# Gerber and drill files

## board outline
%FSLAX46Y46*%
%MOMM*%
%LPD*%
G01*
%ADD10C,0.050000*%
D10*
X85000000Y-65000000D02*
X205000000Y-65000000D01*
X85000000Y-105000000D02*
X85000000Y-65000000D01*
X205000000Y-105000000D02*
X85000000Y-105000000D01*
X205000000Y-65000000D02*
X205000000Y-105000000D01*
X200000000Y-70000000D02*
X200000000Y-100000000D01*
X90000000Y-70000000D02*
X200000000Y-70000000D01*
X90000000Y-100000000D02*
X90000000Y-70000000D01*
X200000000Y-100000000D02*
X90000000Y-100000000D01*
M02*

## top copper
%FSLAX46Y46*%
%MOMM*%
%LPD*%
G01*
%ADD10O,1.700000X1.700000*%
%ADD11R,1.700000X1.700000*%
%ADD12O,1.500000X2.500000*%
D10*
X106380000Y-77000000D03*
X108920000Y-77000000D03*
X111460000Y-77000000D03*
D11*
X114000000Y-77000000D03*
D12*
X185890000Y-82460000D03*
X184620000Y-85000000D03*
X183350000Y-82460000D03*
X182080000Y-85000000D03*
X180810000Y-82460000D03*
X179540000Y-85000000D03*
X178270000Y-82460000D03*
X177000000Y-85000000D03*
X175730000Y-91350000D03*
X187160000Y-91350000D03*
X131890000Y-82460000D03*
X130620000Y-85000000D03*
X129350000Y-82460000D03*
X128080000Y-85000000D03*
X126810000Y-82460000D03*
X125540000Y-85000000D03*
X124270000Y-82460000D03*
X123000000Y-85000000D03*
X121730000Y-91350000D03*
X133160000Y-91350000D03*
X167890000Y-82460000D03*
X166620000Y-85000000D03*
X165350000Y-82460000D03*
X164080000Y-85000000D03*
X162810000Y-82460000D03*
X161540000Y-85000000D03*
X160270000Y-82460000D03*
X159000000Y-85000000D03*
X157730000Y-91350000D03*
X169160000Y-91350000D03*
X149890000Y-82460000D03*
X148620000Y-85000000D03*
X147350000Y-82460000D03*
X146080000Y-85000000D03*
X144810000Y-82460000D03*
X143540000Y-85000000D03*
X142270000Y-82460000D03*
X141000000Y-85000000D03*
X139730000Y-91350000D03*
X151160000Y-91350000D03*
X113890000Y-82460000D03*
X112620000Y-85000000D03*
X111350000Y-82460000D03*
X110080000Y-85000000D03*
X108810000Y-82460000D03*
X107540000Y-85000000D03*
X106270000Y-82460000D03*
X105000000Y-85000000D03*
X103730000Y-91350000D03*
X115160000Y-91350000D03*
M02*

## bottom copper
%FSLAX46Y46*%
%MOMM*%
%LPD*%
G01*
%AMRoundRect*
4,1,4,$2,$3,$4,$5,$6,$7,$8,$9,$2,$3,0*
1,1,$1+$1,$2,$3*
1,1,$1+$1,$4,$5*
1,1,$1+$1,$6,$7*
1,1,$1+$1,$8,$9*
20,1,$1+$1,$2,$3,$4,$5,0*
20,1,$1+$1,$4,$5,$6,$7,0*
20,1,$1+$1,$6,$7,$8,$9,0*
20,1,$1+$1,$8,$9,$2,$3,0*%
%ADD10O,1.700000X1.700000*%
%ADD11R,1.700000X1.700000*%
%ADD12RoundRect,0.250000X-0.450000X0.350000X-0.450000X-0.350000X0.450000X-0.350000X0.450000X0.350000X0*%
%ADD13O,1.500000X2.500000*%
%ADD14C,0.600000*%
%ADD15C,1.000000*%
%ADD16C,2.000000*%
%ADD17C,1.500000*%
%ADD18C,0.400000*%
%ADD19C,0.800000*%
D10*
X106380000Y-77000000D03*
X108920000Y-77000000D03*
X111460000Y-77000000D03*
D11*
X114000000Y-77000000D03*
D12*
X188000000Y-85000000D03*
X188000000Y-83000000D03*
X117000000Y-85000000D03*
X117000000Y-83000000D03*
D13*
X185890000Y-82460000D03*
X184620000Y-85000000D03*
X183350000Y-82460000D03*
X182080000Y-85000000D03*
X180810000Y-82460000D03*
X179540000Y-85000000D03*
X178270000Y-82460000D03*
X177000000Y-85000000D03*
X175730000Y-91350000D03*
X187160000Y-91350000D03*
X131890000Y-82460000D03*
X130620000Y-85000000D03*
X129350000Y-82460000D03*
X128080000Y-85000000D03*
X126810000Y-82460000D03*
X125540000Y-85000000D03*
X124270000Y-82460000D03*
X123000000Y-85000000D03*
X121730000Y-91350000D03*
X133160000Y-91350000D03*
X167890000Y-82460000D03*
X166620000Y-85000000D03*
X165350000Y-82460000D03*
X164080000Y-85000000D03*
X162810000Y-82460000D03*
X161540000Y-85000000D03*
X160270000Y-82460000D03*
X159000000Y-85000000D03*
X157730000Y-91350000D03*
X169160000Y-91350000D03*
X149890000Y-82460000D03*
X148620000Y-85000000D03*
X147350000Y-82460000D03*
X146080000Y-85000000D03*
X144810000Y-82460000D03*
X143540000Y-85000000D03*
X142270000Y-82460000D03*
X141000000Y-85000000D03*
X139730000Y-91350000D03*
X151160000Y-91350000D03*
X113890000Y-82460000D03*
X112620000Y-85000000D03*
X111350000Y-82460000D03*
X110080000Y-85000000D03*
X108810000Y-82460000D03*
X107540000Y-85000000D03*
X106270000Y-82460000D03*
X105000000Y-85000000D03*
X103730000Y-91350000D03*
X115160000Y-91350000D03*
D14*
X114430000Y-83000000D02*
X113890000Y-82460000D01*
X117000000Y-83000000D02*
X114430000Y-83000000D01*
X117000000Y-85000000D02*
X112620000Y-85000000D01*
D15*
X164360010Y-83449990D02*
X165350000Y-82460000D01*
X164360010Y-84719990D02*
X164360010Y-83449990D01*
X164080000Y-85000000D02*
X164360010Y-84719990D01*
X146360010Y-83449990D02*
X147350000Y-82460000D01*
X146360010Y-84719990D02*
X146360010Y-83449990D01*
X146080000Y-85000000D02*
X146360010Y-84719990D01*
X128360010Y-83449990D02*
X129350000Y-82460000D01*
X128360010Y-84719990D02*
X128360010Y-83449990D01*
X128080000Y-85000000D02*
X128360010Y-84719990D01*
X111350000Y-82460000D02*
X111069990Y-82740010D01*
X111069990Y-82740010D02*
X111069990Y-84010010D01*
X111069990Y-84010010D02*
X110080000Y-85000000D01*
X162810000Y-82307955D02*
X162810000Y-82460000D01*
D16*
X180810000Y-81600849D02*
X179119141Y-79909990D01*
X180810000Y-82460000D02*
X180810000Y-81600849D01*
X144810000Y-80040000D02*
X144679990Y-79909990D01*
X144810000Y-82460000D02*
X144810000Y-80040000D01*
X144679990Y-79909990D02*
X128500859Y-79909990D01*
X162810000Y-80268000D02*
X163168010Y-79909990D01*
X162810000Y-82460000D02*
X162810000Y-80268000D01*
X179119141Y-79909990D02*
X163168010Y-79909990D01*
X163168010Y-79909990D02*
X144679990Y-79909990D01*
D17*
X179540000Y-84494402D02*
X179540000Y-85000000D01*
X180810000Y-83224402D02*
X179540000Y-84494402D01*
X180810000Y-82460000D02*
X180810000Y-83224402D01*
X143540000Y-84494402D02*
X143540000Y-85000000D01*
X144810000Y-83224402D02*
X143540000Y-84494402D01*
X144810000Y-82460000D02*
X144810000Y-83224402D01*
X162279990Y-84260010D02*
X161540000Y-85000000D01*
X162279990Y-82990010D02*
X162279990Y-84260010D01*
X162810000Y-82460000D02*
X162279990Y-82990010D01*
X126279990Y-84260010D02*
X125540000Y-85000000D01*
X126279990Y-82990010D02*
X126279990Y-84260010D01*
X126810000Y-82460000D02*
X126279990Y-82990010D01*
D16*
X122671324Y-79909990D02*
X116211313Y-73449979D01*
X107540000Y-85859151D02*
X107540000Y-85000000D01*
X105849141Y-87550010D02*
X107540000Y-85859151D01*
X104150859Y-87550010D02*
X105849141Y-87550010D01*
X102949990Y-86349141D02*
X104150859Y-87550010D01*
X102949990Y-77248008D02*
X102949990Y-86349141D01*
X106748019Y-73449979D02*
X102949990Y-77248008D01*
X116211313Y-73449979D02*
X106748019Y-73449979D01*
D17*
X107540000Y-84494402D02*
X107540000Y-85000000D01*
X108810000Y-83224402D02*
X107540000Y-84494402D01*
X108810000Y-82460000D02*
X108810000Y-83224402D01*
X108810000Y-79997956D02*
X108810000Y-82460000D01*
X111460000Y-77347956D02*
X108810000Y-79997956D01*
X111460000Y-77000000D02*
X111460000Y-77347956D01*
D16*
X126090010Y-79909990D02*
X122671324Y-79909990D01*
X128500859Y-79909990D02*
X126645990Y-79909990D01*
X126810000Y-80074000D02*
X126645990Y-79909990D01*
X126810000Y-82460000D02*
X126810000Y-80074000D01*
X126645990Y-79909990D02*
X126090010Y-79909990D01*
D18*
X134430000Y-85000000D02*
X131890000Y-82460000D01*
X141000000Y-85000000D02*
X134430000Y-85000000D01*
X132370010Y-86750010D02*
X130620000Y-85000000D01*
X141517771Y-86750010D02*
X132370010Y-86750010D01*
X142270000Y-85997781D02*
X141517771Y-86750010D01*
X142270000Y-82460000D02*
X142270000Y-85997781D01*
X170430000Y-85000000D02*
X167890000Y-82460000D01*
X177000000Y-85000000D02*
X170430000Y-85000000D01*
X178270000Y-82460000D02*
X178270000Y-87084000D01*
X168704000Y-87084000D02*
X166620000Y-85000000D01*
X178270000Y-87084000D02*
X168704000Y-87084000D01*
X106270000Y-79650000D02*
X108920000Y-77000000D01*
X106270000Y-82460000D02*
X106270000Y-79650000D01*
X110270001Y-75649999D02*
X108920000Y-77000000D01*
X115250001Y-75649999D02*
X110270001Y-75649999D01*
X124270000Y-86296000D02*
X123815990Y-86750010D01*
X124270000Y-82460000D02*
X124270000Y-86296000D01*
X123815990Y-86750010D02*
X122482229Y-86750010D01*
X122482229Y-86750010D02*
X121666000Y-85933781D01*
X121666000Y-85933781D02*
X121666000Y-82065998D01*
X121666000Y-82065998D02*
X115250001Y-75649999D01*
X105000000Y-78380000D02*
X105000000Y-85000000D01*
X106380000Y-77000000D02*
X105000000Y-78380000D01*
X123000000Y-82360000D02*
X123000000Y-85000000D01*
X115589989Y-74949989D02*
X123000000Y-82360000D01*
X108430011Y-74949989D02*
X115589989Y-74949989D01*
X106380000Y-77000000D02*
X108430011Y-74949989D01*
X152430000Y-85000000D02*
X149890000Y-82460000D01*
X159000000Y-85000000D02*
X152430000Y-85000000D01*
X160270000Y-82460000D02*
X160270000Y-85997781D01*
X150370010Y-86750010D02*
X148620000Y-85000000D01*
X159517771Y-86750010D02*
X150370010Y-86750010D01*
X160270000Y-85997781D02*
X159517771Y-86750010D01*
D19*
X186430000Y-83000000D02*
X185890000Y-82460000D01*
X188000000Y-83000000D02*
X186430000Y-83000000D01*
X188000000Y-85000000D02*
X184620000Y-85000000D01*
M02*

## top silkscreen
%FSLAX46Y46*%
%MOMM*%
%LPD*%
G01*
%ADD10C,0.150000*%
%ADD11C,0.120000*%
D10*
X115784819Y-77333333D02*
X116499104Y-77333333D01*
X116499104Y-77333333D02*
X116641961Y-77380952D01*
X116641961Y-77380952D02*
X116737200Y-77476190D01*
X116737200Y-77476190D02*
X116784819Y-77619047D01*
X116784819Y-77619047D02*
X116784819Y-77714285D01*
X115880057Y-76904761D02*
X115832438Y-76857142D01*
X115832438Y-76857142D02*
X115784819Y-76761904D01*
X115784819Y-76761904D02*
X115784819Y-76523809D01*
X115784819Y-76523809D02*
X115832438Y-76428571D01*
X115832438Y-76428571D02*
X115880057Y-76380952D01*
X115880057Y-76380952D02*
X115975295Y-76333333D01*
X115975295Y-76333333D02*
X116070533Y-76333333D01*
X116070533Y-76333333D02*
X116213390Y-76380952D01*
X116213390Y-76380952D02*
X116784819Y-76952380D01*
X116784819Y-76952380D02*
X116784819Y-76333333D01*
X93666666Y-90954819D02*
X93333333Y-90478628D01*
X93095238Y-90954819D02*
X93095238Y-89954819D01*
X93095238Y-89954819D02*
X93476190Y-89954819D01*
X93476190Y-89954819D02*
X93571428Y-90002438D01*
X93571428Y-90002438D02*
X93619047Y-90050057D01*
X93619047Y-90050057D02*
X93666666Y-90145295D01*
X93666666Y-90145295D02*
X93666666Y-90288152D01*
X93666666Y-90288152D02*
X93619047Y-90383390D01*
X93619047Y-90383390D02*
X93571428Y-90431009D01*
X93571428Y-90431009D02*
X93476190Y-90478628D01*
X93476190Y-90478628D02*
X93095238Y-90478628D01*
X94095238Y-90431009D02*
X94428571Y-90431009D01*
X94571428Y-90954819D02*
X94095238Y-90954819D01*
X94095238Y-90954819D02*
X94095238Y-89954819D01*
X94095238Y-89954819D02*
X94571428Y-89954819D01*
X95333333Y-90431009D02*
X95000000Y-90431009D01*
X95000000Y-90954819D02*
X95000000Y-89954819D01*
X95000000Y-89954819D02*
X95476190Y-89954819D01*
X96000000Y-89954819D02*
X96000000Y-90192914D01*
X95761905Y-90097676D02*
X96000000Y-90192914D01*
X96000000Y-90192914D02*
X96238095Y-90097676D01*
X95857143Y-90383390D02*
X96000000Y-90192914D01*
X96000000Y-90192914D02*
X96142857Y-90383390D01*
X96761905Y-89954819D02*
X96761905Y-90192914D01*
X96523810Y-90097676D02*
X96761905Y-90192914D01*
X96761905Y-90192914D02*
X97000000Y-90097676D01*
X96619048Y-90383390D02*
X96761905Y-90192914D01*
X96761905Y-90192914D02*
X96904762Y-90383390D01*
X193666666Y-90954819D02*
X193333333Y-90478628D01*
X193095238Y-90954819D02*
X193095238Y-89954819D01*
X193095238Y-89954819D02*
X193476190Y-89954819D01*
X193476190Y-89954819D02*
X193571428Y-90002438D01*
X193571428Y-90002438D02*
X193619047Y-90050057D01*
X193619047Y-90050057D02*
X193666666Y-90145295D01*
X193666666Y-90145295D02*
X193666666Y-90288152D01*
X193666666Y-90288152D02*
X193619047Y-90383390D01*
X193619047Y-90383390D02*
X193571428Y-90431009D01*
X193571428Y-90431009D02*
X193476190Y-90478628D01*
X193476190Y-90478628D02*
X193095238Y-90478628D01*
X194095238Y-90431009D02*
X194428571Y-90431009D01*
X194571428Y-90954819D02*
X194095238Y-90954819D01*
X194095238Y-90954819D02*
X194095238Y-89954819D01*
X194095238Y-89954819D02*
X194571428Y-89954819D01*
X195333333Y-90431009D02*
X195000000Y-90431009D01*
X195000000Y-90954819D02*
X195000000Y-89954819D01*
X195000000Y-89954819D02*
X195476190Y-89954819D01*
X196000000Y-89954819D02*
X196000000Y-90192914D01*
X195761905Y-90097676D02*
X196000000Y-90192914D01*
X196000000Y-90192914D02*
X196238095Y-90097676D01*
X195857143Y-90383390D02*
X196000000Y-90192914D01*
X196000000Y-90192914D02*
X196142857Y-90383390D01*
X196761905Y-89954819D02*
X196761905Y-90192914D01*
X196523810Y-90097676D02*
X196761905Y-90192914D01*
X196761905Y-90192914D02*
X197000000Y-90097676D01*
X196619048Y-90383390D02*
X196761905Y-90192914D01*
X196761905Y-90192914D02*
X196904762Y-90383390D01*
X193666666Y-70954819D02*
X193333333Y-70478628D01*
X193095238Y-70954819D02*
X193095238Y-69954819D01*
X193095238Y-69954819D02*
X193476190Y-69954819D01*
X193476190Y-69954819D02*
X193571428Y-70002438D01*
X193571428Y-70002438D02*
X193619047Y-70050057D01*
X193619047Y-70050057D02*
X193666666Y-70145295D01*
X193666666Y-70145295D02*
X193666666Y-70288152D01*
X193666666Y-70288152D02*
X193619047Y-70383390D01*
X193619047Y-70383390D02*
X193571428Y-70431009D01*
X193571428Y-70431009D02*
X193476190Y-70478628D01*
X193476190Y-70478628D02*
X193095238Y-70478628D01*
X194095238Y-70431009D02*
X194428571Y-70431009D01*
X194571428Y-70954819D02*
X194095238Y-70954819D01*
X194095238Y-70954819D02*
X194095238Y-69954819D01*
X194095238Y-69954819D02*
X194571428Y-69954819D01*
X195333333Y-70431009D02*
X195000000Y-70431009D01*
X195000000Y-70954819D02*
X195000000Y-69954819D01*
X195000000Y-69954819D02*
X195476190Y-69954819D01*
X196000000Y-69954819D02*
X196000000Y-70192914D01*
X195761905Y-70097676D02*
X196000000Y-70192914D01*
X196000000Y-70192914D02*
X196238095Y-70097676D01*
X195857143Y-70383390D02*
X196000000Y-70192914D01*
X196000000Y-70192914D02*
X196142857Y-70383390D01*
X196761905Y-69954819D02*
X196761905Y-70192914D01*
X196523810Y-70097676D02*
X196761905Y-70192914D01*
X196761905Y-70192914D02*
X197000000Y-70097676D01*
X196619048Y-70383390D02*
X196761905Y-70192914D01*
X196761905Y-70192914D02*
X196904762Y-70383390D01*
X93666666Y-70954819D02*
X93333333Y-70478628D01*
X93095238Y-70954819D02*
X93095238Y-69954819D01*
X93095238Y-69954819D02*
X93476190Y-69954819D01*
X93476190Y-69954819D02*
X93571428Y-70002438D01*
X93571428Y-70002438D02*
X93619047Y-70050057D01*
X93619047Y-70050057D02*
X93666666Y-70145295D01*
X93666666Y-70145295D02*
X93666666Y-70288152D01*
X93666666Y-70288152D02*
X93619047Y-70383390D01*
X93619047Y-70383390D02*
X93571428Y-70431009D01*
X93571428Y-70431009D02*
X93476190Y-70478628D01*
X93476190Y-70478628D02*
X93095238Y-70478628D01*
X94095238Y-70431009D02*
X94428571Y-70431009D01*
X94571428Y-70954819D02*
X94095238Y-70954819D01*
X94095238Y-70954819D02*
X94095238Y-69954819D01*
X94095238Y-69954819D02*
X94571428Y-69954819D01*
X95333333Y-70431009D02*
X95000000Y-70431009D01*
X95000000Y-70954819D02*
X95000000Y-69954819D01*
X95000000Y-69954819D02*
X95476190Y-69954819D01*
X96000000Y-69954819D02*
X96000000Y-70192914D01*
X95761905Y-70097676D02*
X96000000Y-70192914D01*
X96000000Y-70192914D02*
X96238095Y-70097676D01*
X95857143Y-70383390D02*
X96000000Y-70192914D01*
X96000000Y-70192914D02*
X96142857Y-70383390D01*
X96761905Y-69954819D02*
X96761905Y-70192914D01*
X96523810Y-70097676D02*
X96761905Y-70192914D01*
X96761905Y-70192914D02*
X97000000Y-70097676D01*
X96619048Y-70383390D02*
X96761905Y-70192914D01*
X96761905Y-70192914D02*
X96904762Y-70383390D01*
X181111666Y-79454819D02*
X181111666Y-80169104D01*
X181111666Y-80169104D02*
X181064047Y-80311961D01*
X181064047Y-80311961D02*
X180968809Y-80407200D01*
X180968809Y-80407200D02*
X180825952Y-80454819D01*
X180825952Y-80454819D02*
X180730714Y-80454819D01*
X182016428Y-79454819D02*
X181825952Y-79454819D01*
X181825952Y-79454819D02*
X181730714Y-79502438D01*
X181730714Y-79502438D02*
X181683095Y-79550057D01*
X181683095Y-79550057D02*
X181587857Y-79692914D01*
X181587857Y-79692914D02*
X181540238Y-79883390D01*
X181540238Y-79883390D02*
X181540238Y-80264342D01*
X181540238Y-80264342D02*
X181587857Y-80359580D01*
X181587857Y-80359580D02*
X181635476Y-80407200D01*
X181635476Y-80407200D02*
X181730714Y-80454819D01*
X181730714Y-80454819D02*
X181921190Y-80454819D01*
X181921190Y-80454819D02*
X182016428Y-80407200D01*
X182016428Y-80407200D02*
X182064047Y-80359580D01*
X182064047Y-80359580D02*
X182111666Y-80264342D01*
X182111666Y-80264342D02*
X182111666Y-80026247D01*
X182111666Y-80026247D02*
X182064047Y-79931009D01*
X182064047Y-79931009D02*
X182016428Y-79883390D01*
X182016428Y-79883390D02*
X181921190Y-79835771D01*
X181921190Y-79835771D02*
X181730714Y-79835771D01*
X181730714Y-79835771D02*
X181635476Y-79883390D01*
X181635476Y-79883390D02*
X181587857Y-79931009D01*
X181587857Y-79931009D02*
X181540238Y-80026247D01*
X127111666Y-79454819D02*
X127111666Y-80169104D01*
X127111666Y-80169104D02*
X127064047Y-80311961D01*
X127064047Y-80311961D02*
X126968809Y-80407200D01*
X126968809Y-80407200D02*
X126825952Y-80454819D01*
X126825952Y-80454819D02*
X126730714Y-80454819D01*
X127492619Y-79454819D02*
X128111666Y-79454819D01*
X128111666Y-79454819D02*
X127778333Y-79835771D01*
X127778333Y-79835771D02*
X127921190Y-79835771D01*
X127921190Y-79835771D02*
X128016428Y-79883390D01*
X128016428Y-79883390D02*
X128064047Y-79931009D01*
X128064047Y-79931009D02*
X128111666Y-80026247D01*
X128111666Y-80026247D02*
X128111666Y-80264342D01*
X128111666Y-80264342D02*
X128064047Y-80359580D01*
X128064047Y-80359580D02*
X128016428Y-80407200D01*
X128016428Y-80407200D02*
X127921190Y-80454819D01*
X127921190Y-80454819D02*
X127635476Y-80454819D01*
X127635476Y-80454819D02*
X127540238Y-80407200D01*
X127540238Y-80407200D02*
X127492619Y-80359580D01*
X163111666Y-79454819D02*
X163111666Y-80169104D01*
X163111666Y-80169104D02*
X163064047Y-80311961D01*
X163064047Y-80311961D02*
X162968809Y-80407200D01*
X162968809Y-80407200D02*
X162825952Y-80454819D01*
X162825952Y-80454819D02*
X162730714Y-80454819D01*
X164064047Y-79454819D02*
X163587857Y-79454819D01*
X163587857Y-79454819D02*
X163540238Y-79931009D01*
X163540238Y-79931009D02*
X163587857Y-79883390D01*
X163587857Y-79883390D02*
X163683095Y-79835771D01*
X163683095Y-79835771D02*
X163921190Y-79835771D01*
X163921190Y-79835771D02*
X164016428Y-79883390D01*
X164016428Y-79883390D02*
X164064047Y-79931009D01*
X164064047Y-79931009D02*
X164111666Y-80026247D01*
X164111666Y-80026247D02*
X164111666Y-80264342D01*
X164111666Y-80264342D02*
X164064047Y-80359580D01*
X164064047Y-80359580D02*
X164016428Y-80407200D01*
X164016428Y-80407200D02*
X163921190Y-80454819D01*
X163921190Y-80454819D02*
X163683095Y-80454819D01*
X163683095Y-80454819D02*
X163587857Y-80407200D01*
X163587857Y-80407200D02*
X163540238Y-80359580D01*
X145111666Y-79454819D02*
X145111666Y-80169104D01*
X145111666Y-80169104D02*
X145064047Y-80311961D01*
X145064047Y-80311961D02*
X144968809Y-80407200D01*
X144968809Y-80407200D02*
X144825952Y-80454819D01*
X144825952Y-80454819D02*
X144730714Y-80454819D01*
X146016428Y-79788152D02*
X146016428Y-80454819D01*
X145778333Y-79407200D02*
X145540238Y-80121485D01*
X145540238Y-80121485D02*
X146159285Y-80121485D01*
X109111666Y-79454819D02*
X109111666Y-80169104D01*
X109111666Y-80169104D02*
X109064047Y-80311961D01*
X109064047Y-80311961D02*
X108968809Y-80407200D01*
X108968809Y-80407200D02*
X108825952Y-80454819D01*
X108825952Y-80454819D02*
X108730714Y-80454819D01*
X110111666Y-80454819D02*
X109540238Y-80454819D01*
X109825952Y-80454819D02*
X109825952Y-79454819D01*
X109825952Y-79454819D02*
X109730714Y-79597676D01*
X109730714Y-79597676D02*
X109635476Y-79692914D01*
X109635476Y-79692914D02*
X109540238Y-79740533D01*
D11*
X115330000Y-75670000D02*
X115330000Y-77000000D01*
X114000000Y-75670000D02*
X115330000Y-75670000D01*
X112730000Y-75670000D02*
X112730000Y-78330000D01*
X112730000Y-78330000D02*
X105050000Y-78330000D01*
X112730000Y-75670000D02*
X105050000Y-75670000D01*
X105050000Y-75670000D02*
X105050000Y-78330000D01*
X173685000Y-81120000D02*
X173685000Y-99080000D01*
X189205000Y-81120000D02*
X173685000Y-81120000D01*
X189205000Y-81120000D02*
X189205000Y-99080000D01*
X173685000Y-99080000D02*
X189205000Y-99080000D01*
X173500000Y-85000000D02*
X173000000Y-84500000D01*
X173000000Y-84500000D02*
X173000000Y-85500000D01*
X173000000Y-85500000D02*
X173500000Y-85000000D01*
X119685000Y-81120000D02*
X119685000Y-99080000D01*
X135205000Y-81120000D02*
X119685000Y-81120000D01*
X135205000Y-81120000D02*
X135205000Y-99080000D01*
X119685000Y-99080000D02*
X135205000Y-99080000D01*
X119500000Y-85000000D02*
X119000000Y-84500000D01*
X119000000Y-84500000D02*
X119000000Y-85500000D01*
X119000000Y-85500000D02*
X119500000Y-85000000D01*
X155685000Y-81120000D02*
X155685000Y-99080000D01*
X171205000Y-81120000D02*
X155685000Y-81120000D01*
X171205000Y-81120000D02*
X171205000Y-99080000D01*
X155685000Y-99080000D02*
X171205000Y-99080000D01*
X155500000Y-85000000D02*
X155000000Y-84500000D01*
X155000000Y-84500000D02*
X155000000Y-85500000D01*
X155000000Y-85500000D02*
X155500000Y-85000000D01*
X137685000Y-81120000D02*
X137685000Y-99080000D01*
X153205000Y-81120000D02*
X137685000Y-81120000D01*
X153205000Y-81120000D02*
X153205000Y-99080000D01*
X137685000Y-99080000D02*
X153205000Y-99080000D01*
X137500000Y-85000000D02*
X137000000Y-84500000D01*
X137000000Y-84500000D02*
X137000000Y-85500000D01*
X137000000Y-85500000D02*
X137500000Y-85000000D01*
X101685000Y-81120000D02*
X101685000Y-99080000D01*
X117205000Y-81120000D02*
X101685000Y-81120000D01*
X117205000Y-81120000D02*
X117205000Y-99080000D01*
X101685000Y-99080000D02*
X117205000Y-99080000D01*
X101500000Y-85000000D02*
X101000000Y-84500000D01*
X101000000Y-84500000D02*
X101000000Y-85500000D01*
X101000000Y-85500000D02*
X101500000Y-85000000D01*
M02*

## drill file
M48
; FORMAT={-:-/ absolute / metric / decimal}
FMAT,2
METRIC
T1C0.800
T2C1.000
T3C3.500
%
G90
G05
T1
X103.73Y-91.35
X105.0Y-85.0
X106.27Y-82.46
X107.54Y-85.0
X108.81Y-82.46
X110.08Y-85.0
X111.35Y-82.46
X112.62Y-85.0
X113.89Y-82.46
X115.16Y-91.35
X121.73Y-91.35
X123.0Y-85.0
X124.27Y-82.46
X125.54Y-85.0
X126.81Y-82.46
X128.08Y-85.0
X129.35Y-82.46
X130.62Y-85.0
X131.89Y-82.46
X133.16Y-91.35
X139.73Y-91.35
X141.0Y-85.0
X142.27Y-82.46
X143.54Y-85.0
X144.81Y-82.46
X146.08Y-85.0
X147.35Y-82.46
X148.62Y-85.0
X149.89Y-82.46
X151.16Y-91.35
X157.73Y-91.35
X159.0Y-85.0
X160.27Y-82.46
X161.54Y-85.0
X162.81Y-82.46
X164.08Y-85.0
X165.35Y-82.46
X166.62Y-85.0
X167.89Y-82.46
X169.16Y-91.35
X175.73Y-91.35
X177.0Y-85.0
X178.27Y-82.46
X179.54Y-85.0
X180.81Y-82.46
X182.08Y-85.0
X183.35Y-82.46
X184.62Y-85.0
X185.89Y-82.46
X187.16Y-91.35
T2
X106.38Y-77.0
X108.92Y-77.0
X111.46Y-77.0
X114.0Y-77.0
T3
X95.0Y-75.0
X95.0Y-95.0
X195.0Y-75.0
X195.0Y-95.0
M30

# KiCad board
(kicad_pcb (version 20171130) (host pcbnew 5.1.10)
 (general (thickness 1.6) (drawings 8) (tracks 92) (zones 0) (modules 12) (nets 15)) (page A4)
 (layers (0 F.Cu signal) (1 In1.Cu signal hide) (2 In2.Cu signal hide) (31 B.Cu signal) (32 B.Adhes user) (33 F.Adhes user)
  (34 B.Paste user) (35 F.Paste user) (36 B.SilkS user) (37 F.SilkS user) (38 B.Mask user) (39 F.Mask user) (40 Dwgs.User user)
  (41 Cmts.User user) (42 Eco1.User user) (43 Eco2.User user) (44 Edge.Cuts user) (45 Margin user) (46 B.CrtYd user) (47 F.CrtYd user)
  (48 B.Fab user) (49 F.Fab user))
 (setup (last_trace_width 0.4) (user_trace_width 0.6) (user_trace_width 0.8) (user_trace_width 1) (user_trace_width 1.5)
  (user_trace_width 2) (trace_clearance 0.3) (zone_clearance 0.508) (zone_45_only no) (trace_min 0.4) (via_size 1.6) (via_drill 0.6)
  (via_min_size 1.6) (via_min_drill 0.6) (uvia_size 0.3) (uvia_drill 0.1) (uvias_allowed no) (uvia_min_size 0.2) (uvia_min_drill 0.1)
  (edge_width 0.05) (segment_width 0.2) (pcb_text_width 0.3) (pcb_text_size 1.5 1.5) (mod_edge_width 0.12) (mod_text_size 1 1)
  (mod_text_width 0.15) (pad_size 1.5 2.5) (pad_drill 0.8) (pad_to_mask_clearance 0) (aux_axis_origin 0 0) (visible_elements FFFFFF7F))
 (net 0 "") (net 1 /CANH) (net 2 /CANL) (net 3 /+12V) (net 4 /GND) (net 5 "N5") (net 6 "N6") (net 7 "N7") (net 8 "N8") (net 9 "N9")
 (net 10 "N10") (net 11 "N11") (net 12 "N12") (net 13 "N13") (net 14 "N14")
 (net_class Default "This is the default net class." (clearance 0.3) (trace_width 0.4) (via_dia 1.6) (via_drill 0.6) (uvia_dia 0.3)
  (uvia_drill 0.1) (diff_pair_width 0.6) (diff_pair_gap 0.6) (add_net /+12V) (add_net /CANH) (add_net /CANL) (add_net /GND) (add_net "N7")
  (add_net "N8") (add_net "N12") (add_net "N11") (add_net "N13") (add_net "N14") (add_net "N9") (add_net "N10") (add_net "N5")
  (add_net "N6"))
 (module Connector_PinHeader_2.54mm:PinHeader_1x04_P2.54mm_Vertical (layer F.Cu) (at 114 77 270)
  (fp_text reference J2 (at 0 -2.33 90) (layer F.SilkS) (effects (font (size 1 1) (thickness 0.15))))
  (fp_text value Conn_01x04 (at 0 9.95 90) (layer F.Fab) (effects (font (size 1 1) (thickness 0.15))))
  (fp_line (start -1.33 -1.33) (end 0 -1.33) (layer F.SilkS) (width 0.12))
  (fp_line (start -1.33 0) (end -1.33 -1.33) (layer F.SilkS) (width 0.12))
  (fp_line (start -1.33 1.27) (end 1.33 1.27) (layer F.SilkS) (width 0.12))
  (fp_line (start 1.33 1.27) (end 1.33 8.95) (layer F.SilkS) (width 0.12))
  (fp_line (start -1.33 1.27) (end -1.33 8.95) (layer F.SilkS) (width 0.12))
  (fp_line (start -1.33 8.95) (end 1.33 8.95) (layer F.SilkS) (width 0.12))
  (pad 4 thru_hole oval (at 0 7.62 270) (size 1.7 1.7) (drill 1) (layers *.Cu *.Mask) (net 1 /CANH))
  (pad 3 thru_hole oval (at 0 5.08 270) (size 1.7 1.7) (drill 1) (layers *.Cu *.Mask) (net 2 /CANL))
  (pad 2 thru_hole oval (at 0 2.54 270) (size 1.7 1.7) (drill 1) (layers *.Cu *.Mask) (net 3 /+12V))
  (pad 1 thru_hole rect (at 0 0 270) (size 1.7 1.7) (drill 1) (layers *.Cu *.Mask) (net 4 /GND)))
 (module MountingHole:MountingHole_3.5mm (layer F.Cu) (at 95 95)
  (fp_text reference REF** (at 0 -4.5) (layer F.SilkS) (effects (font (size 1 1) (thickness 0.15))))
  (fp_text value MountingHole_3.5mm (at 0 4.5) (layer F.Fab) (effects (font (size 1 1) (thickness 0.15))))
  (pad 1 np_thru_hole circle (at 0 0) (size 3.5 3.5) (drill 3.5) (layers *.Cu *.Mask)))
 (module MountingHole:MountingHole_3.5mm (layer F.Cu) (at 195 95)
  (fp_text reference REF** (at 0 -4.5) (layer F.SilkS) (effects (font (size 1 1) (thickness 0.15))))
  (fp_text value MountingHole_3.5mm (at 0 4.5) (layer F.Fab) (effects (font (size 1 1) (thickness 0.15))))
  (pad 1 np_thru_hole circle (at 0 0) (size 3.5 3.5) (drill 3.5) (layers *.Cu *.Mask)))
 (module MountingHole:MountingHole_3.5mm (layer F.Cu) (at 195 75)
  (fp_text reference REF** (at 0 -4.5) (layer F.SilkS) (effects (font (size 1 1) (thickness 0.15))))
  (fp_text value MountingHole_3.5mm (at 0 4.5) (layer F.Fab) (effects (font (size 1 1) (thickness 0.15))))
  (pad 1 np_thru_hole circle (at 0 0) (size 3.5 3.5) (drill 3.5) (layers *.Cu *.Mask)))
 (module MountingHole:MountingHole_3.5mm (layer F.Cu) (at 95 75)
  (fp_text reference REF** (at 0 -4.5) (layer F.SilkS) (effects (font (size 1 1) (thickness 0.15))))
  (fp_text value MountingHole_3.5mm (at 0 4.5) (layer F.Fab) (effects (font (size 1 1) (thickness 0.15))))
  (pad 1 np_thru_hole circle (at 0 0) (size 3.5 3.5) (drill 3.5) (layers *.Cu *.Mask)))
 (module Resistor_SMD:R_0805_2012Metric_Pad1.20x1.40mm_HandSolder (layer B.Cu) (at 188 84 270)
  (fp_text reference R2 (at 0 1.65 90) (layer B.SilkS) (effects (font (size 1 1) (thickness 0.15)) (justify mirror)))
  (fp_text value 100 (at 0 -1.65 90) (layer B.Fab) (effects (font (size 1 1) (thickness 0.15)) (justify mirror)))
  (pad 2 smd roundrect (at 1 0 270) (size 1.2 1.4) (layers B.Cu B.Paste B.Mask) (roundrect_rratio 0.208333) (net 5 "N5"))
  (pad 1 smd roundrect (at -1 0 270) (size 1.2 1.4) (layers B.Cu B.Paste B.Mask) (roundrect_rratio 0.208333) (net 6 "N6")))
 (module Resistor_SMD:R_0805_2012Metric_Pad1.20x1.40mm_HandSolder (layer B.Cu) (at 117 84 270)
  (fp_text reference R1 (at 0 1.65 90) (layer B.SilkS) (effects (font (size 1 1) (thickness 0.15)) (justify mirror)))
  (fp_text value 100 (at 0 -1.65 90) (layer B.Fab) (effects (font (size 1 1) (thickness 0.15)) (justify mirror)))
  (pad 2 smd roundrect (at 1 0 270) (size 1.2 1.4) (layers B.Cu B.Paste B.Mask) (roundrect_rratio 0.208333) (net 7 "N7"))
  (pad 1 smd roundrect (at -1 0 270) (size 1.2 1.4) (layers B.Cu B.Paste B.Mask) (roundrect_rratio 0.208333) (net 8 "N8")))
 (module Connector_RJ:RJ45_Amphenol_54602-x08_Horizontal (layer F.Cu) (at 177 85)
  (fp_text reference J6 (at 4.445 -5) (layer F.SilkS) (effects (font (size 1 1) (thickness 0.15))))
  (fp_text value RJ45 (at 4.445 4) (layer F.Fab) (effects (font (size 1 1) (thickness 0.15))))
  (fp_line (start -3.315 -3.88) (end -3.315 14.08) (layer F.SilkS) (width 0.12))
  (fp_line (start 12.205 -3.88) (end -3.315 -3.88) (layer F.SilkS) (width 0.12))
  (fp_line (start 12.205 -3.88) (end 12.205 14.08) (layer F.SilkS) (width 0.12))
  (fp_line (start -3.315 14.08) (end 12.205 14.08) (layer F.SilkS) (width 0.12))
  (fp_line (start -3.5 0) (end -4 -0.5) (layer F.SilkS) (width 0.12))
  (fp_line (start -4 -0.5) (end -4 0.5) (layer F.SilkS) (width 0.12))
  (fp_line (start -4 0.5) (end -3.5 0) (layer F.SilkS) (width 0.12))
  (pad 8 thru_hole oval (at 8.89 -2.54) (size 1.5 2.5) (drill 0.8) (layers *.Cu *.Mask) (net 6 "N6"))
  (pad 7 thru_hole oval (at 7.62 0) (size 1.5 2.5) (drill 0.8) (layers *.Cu *.Mask) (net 5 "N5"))
  (pad 6 thru_hole oval (at 6.35 -2.54) (size 1.5 2.5) (drill 0.8) (layers *.Cu *.Mask) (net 4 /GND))
  (pad 5 thru_hole oval (at 5.08 0) (size 1.5 2.5) (drill 0.8) (layers *.Cu *.Mask) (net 4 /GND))
  (pad 4 thru_hole oval (at 3.81 -2.54) (size 1.5 2.5) (drill 0.8) (layers *.Cu *.Mask) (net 3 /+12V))
  (pad 3 thru_hole oval (at 2.54 0) (size 1.5 2.5) (drill 0.8) (layers *.Cu *.Mask) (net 3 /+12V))
  (pad 2 thru_hole oval (at 1.27 -2.54) (size 1.5 2.5) (drill 0.8) (layers *.Cu *.Mask) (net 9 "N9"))
  (pad 1 thru_hole oval (at 0 0) (size 1.5 2.5) (drill 0.8) (layers *.Cu *.Mask) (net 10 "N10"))
  (pad "" thru_hole oval (at -1.27 6.35) (size 1.5 2.5) (drill 0.8) (layers *.Cu *.Mask))
  (pad "" thru_hole oval (at 10.16 6.35) (size 1.5 2.5) (drill 0.8) (layers *.Cu *.Mask)))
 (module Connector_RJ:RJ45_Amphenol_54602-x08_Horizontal (layer F.Cu) (at 123 85)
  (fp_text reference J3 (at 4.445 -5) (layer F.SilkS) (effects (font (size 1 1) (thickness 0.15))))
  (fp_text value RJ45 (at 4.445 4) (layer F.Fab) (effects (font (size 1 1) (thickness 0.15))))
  (fp_line (start -3.315 -3.88) (end -3.315 14.08) (layer F.SilkS) (width 0.12))
  (fp_line (start 12.205 -3.88) (end -3.315 -3.88) (layer F.SilkS) (width 0.12))
  (fp_line (start 12.205 -3.88) (end 12.205 14.08) (layer F.SilkS) (width 0.12))
  (fp_line (start -3.315 14.08) (end 12.205 14.08) (layer F.SilkS) (width 0.12))
  (fp_line (start -3.5 0) (end -4 -0.5) (layer F.SilkS) (width 0.12))
  (fp_line (start -4 -0.5) (end -4 0.5) (layer F.SilkS) (width 0.12))
  (fp_line (start -4 0.5) (end -3.5 0) (layer F.SilkS) (width 0.12))
  (pad 8 thru_hole oval (at 8.89 -2.54) (size 1.5 2.5) (drill 0.8) (layers *.Cu *.Mask) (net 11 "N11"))
  (pad 7 thru_hole oval (at 7.62 0) (size 1.5 2.5) (drill 0.8) (layers *.Cu *.Mask) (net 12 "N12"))
  (pad 6 thru_hole oval (at 6.35 -2.54) (size 1.5 2.5) (drill 0.8) (layers *.Cu *.Mask) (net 4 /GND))
  (pad 5 thru_hole oval (at 5.08 0) (size 1.5 2.5) (drill 0.8) (layers *.Cu *.Mask) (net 4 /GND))
  (pad 4 thru_hole oval (at 3.81 -2.54) (size 1.5 2.5) (drill 0.8) (layers *.Cu *.Mask) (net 3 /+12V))
  (pad 3 thru_hole oval (at 2.54 0) (size 1.5 2.5) (drill 0.8) (layers *.Cu *.Mask) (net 3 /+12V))
  (pad 2 thru_hole oval (at 1.27 -2.54) (size 1.5 2.5) (drill 0.8) (layers *.Cu *.Mask) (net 2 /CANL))
  (pad 1 thru_hole oval (at 0 0) (size 1.5 2.5) (drill 0.8) (layers *.Cu *.Mask) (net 1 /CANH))
  (pad "" thru_hole oval (at -1.27 6.35) (size 1.5 2.5) (drill 0.8) (layers *.Cu *.Mask))
  (pad "" thru_hole oval (at 10.16 6.35) (size 1.5 2.5) (drill 0.8) (layers *.Cu *.Mask)))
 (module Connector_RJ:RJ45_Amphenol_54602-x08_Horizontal (layer F.Cu) (at 159 85)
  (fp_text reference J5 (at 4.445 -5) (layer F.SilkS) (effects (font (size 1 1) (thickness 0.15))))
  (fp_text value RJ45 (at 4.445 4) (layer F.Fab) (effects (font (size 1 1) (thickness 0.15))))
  (fp_line (start -3.315 -3.88) (end -3.315 14.08) (layer F.SilkS) (width 0.12))
  (fp_line (start 12.205 -3.88) (end -3.315 -3.88) (layer F.SilkS) (width 0.12))
  (fp_line (start 12.205 -3.88) (end 12.205 14.08) (layer F.SilkS) (width 0.12))
  (fp_line (start -3.315 14.08) (end 12.205 14.08) (layer F.SilkS) (width 0.12))
  (fp_line (start -3.5 0) (end -4 -0.5) (layer F.SilkS) (width 0.12))
  (fp_line (start -4 -0.5) (end -4 0.5) (layer F.SilkS) (width 0.12))
  (fp_line (start -4 0.5) (end -3.5 0) (layer F.SilkS) (width 0.12))
  (pad 8 thru_hole oval (at 8.89 -2.54) (size 1.5 2.5) (drill 0.8) (layers *.Cu *.Mask) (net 10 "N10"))
  (pad 7 thru_hole oval (at 7.62 0) (size 1.5 2.5) (drill 0.8) (layers *.Cu *.Mask) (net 9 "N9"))
  (pad 6 thru_hole oval (at 6.35 -2.54) (size 1.5 2.5) (drill 0.8) (layers *.Cu *.Mask) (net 4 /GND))
  (pad 5 thru_hole oval (at 5.08 0) (size 1.5 2.5) (drill 0.8) (layers *.Cu *.Mask) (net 4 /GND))
  (pad 4 thru_hole oval (at 3.81 -2.54) (size 1.5 2.5) (drill 0.8) (layers *.Cu *.Mask) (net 3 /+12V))
  (pad 3 thru_hole oval (at 2.54 0) (size 1.5 2.5) (drill 0.8) (layers *.Cu *.Mask) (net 3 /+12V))
  (pad 2 thru_hole oval (at 1.27 -2.54) (size 1.5 2.5) (drill 0.8) (layers *.Cu *.Mask) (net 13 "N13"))
  (pad 1 thru_hole oval (at 0 0) (size 1.5 2.5) (drill 0.8) (layers *.Cu *.Mask) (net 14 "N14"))
  (pad "" thru_hole oval (at -1.27 6.35) (size 1.5 2.5) (drill 0.8) (layers *.Cu *.Mask))
  (pad "" thru_hole oval (at 10.16 6.35) (size 1.5 2.5) (drill 0.8) (layers *.Cu *.Mask)))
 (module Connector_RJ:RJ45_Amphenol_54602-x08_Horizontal (layer F.Cu) (at 141 85)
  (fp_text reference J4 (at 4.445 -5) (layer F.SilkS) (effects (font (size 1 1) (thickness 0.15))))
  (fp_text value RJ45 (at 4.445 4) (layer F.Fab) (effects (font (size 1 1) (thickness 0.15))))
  (fp_line (start -3.315 -3.88) (end -3.315 14.08) (layer F.SilkS) (width 0.12))
  (fp_line (start 12.205 -3.88) (end -3.315 -3.88) (layer F.SilkS) (width 0.12))
  (fp_line (start 12.205 -3.88) (end 12.205 14.08) (layer F.SilkS) (width 0.12))
  (fp_line (start -3.315 14.08) (end 12.205 14.08) (layer F.SilkS) (width 0.12))
  (fp_line (start -3.5 0) (end -4 -0.5) (layer F.SilkS) (width 0.12))
  (fp_line (start -4 -0.5) (end -4 0.5) (layer F.SilkS) (width 0.12))
  (fp_line (start -4 0.5) (end -3.5 0) (layer F.SilkS) (width 0.12))
  (pad 8 thru_hole oval (at 8.89 -2.54) (size 1.5 2.5) (drill 0.8) (layers *.Cu *.Mask) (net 14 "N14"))
  (pad 7 thru_hole oval (at 7.62 0) (size 1.5 2.5) (drill 0.8) (layers *.Cu *.Mask) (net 13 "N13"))
  (pad 6 thru_hole oval (at 6.35 -2.54) (size 1.5 2.5) (drill 0.8) (layers *.Cu *.Mask) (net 4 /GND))
  (pad 5 thru_hole oval (at 5.08 0) (size 1.5 2.5) (drill 0.8) (layers *.Cu *.Mask) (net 4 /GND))
  (pad 4 thru_hole oval (at 3.81 -2.54) (size 1.5 2.5) (drill 0.8) (layers *.Cu *.Mask) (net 3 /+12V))
  (pad 3 thru_hole oval (at 2.54 0) (size 1.5 2.5) (drill 0.8) (layers *.Cu *.Mask) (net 3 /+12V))
  (pad 2 thru_hole oval (at 1.27 -2.54) (size 1.5 2.5) (drill 0.8) (layers *.Cu *.Mask) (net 12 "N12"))
  (pad 1 thru_hole oval (at 0 0) (size 1.5 2.5) (drill 0.8) (layers *.Cu *.Mask) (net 11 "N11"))
  (pad "" thru_hole oval (at -1.27 6.35) (size 1.5 2.5) (drill 0.8) (layers *.Cu *.Mask))
  (pad "" thru_hole oval (at 10.16 6.35) (size 1.5 2.5) (drill 0.8) (layers *.Cu *.Mask)))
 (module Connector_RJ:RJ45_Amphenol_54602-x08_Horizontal (layer F.Cu) (at 105 85)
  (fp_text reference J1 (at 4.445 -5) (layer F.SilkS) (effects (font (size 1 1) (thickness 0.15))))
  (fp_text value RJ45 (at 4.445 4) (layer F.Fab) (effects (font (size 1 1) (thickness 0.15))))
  (fp_line (start -3.315 -3.88) (end -3.315 14.08) (layer F.SilkS) (width 0.12))
  (fp_line (start 12.205 -3.88) (end -3.315 -3.88) (layer F.SilkS) (width 0.12))
  (fp_line (start 12.205 -3.88) (end 12.205 14.08) (layer F.SilkS) (width 0.12))
  (fp_line (start -3.315 14.08) (end 12.205 14.08) (layer F.SilkS) (width 0.12))
  (fp_line (start -3.5 0) (end -4 -0.5) (layer F.SilkS) (width 0.12))
  (fp_line (start -4 -0.5) (end -4 0.5) (layer F.SilkS) (width 0.12))
  (fp_line (start -4 0.5) (end -3.5 0) (layer F.SilkS) (width 0.12))
  (pad 8 thru_hole oval (at 8.89 -2.54) (size 1.5 2.5) (drill 0.8) (layers *.Cu *.Mask) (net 8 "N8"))
  (pad 7 thru_hole oval (at 7.62 0) (size 1.5 2.5) (drill 0.8) (layers *.Cu *.Mask) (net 7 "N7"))
  (pad 6 thru_hole oval (at 6.35 -2.54) (size 1.5 2.5) (drill 0.8) (layers *.Cu *.Mask) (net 4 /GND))
  (pad 5 thru_hole oval (at 5.08 0) (size 1.5 2.5) (drill 0.8) (layers *.Cu *.Mask) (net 4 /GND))
  (pad 4 thru_hole oval (at 3.81 -2.54) (size 1.5 2.5) (drill 0.8) (layers *.Cu *.Mask) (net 3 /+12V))
  (pad 3 thru_hole oval (at 2.54 0) (size 1.5 2.5) (drill 0.8) (layers *.Cu *.Mask) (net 3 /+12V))
  (pad 2 thru_hole oval (at 1.27 -2.54) (size 1.5 2.5) (drill 0.8) (layers *.Cu *.Mask) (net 2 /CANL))
  (pad 1 thru_hole oval (at 0 0) (size 1.5 2.5) (drill 0.8) (layers *.Cu *.Mask) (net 1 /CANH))
  (pad "" thru_hole oval (at -1.27 6.35) (size 1.5 2.5) (drill 0.8) (layers *.Cu *.Mask))
  (pad "" thru_hole oval (at 10.16 6.35) (size 1.5 2.5) (drill 0.8) (layers *.Cu *.Mask)))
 (gr_line (start 85 65) (end 205 65) (layer Edge.Cuts) (width 0.05))
 (gr_line (start 85 105) (end 85 65) (layer Edge.Cuts) (width 0.05))
 (gr_line (start 205 105) (end 85 105) (layer Edge.Cuts) (width 0.05))
 (gr_line (start 205 65) (end 205 105) (layer Edge.Cuts) (width 0.05))
 (gr_line (start 200 70) (end 200 100) (layer Edge.Cuts) (width 0.05))
 (gr_line (start 90 70) (end 200 70) (layer Edge.Cuts) (width 0.05))
 (gr_line (start 90 100) (end 90 70) (layer Edge.Cuts) (width 0.05))
 (gr_line (start 200 100) (end 90 100) (layer Edge.Cuts) (width 0.05))
 (segment (start 114.43 83) (end 113.89 82.46) (width 0.6) (layer B.Cu) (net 8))
 (segment (start 117 83) (end 114.43 83) (width 0.6) (layer B.Cu) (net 8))
 (segment (start 117 85) (end 112.62 85) (width 0.6) (layer B.Cu) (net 7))
 (segment (start 164.36001 83.44999) (end 165.35 82.46) (width 1) (layer B.Cu) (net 4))
 (segment (start 164.36001 84.71999) (end 164.36001 83.44999) (width 1) (layer B.Cu) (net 4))
 (segment (start 164.08 85) (end 164.36001 84.71999) (width 1) (layer B.Cu) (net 4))
 (segment (start 146.36001 83.44999) (end 147.35 82.46) (width 1) (layer B.Cu) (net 4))
 (segment (start 146.36001 84.71999) (end 146.36001 83.44999) (width 1) (layer B.Cu) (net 4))
 (segment (start 146.08 85) (end 146.36001 84.71999) (width 1) (layer B.Cu) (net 4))
 (segment (start 128.36001 83.44999) (end 129.35 82.46) (width 1) (layer B.Cu) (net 4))
 (segment (start 128.36001 84.71999) (end 128.36001 83.44999) (width 1) (layer B.Cu) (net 4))
 (segment (start 128.08 85) (end 128.36001 84.71999) (width 1) (layer B.Cu) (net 4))
 (segment (start 111.35 82.46) (end 111.06999 82.74001) (width 1) (layer B.Cu) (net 4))
 (segment (start 111.06999 82.74001) (end 111.06999 84.01001) (width 1) (layer B.Cu) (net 4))
 (segment (start 111.06999 84.01001) (end 110.08 85) (width 1) (layer B.Cu) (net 4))
 (segment (start 162.81 82.307955) (end 162.81 82.46) (width 1) (layer B.Cu) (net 3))
 (segment (start 180.81 81.600849) (end 179.119141 79.90999) (width 2) (layer B.Cu) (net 3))
 (segment (start 180.81 82.46) (end 180.81 81.600849) (width 2) (layer B.Cu) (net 3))
 (segment (start 144.81 80.04) (end 144.67999 79.90999) (width 2) (layer B.Cu) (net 3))
 (segment (start 144.81 82.46) (end 144.81 80.04) (width 2) (layer B.Cu) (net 3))
 (segment (start 144.67999 79.90999) (end 128.500859 79.90999) (width 2) (layer B.Cu) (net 3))
 (segment (start 162.81 80.268) (end 163.16801 79.90999) (width 2) (layer B.Cu) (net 3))
 (segment (start 162.81 82.46) (end 162.81 80.268) (width 2) (layer B.Cu) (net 3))
 (segment (start 179.119141 79.90999) (end 163.16801 79.90999) (width 2) (layer B.Cu) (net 3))
 (segment (start 163.16801 79.90999) (end 144.67999 79.90999) (width 2) (layer B.Cu) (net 3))
 (segment (start 179.54 84.494402) (end 179.54 85) (width 1.5) (layer B.Cu) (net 3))
 (segment (start 180.81 83.224402) (end 179.54 84.494402) (width 1.5) (layer B.Cu) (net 3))
 (segment (start 180.81 82.46) (end 180.81 83.224402) (width 1.5) (layer B.Cu) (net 3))
 (segment (start 143.54 84.494402) (end 143.54 85) (width 1.5) (layer B.Cu) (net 3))
 (segment (start 144.81 83.224402) (end 143.54 84.494402) (width 1.5) (layer B.Cu) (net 3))
 (segment (start 144.81 82.46) (end 144.81 83.224402) (width 1.5) (layer B.Cu) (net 3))
 (segment (start 162.27999 84.26001) (end 161.54 85) (width 1.5) (layer B.Cu) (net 3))
 (segment (start 162.27999 82.99001) (end 162.27999 84.26001) (width 1.5) (layer B.Cu) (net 3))
 (segment (start 162.81 82.46) (end 162.27999 82.99001) (width 1.5) (layer B.Cu) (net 3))
 (segment (start 126.27999 84.26001) (end 125.54 85) (width 1.5) (layer B.Cu) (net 3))
 (segment (start 126.27999 82.99001) (end 126.27999 84.26001) (width 1.5) (layer B.Cu) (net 3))
 (segment (start 126.81 82.46) (end 126.27999 82.99001) (width 1.5) (layer B.Cu) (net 3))
 (segment (start 122.671324 79.90999) (end 116.211313 73.449979) (width 2) (layer B.Cu) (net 3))
 (segment (start 107.54 85.859151) (end 107.54 85) (width 2) (layer B.Cu) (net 3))
 (segment (start 105.849141 87.55001) (end 107.54 85.859151) (width 2) (layer B.Cu) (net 3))
 (segment (start 104.150859 87.55001) (end 105.849141 87.55001) (width 2) (layer B.Cu) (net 3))
 (segment (start 102.94999 86.349141) (end 104.150859 87.55001) (width 2) (layer B.Cu) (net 3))
 (segment (start 102.94999 77.248008) (end 102.94999 86.349141) (width 2) (layer B.Cu) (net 3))
 (segment (start 106.748019 73.449979) (end 102.94999 77.248008) (width 2) (layer B.Cu) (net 3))
 (segment (start 116.211313 73.449979) (end 106.748019 73.449979) (width 2) (layer B.Cu) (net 3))
 (segment (start 107.54 84.494402) (end 107.54 85) (width 1.5) (layer B.Cu) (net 3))
 (segment (start 108.81 83.224402) (end 107.54 84.494402) (width 1.5) (layer B.Cu) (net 3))
 (segment (start 108.81 82.46) (end 108.81 83.224402) (width 1.5) (layer B.Cu) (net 3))
 (segment (start 108.81 79.997956) (end 108.81 82.46) (width 1.5) (layer B.Cu) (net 3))
 (segment (start 111.46 77.347956) (end 108.81 79.997956) (width 1.5) (layer B.Cu) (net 3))
 (segment (start 111.46 77) (end 111.46 77.347956) (width 1.5) (layer B.Cu) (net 3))
 (segment (start 126.09001 79.90999) (end 122.671324 79.90999) (width 2) (layer B.Cu) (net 3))
 (segment (start 128.500859 79.90999) (end 126.64599 79.90999) (width 2) (layer B.Cu) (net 3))
 (segment (start 126.81 80.074) (end 126.64599 79.90999) (width 2) (layer B.Cu) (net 3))
 (segment (start 126.81 82.46) (end 126.81 80.074) (width 2) (layer B.Cu) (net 3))
 (segment (start 126.64599 79.90999) (end 126.09001 79.90999) (width 2) (layer B.Cu) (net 3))
 (segment (start 134.43 85) (end 131.89 82.46) (width 0.4) (layer B.Cu) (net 11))
 (segment (start 141 85) (end 134.43 85) (width 0.4) (layer B.Cu) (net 11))
 (segment (start 132.37001 86.75001) (end 130.62 85) (width 0.4) (layer B.Cu) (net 12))
 (segment (start 141.517771 86.75001) (end 132.37001 86.75001) (width 0.4) (layer B.Cu) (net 12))
 (segment (start 142.27 85.997781) (end 141.517771 86.75001) (width 0.4) (layer B.Cu) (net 12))
 (segment (start 142.27 82.46) (end 142.27 85.997781) (width 0.4) (layer B.Cu) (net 12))
 (segment (start 170.43 85) (end 167.89 82.46) (width 0.4) (layer B.Cu) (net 10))
 (segment (start 177 85) (end 170.43 85) (width 0.4) (layer B.Cu) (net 10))
 (segment (start 178.27 82.46) (end 178.27 87.084) (width 0.4) (layer B.Cu) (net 9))
 (segment (start 168.704 87.084) (end 166.62 85) (width 0.4) (layer B.Cu) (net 9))
 (segment (start 178.27 87.084) (end 168.704 87.084) (width 0.4) (layer B.Cu) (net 9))
 (segment (start 106.27 79.65) (end 108.92 77) (width 0.4) (layer B.Cu) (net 2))
 (segment (start 106.27 82.46) (end 106.27 79.65) (width 0.4) (layer B.Cu) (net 2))
 (segment (start 110.270001 75.649999) (end 108.92 77) (width 0.4) (layer B.Cu) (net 2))
 (segment (start 115.250001 75.649999) (end 110.270001 75.649999) (width 0.4) (layer B.Cu) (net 2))
 (segment (start 124.27 86.296) (end 123.81599 86.75001) (width 0.4) (layer B.Cu) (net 2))
 (segment (start 124.27 82.46) (end 124.27 86.296) (width 0.4) (layer B.Cu) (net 2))
 (segment (start 123.81599 86.75001) (end 122.482229 86.75001) (width 0.4) (layer B.Cu) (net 2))
 (segment (start 122.482229 86.75001) (end 121.666 85.933781) (width 0.4) (layer B.Cu) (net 2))
 (segment (start 121.666 85.933781) (end 121.666 82.065998) (width 0.4) (layer B.Cu) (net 2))
 (segment (start 121.666 82.065998) (end 115.250001 75.649999) (width 0.4) (layer B.Cu) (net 2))
 (segment (start 105 78.38) (end 105 85) (width 0.4) (layer B.Cu) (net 1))
 (segment (start 106.38 77) (end 105 78.38) (width 0.4) (layer B.Cu) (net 1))
 (segment (start 123 82.36) (end 123 85) (width 0.4) (layer B.Cu) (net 1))
 (segment (start 115.589989 74.949989) (end 123 82.36) (width 0.4) (layer B.Cu) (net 1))
 (segment (start 108.430011 74.949989) (end 115.589989 74.949989) (width 0.4) (layer B.Cu) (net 1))
 (segment (start 106.38 77) (end 108.430011 74.949989) (width 0.4) (layer B.Cu) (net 1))
 (segment (start 152.43 85) (end 149.89 82.46) (width 0.4) (layer B.Cu) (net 14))
 (segment (start 159 85) (end 152.43 85) (width 0.4) (layer B.Cu) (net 14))
 (segment (start 160.27 82.46) (end 160.27 85.997781) (width 0.4) (layer B.Cu) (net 13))
 (segment (start 150.37001 86.75001) (end 148.62 85) (width 0.4) (layer B.Cu) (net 13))
 (segment (start 159.517771 86.75001) (end 150.37001 86.75001) (width 0.4) (layer B.Cu) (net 13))
 (segment (start 160.27 85.997781) (end 159.517771 86.75001) (width 0.4) (layer B.Cu) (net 13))
 (segment (start 186.43 83) (end 185.89 82.46) (width 0.8) (layer B.Cu) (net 6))
 (segment (start 188 83) (end 186.43 83) (width 0.8) (layer B.Cu) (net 6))
 (segment (start 188 85) (end 184.62 85) (width 0.8) (layer B.Cu) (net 5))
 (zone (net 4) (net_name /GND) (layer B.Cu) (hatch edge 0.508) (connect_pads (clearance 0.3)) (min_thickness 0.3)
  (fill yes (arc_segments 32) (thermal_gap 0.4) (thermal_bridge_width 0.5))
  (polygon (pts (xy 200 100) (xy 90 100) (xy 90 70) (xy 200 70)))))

